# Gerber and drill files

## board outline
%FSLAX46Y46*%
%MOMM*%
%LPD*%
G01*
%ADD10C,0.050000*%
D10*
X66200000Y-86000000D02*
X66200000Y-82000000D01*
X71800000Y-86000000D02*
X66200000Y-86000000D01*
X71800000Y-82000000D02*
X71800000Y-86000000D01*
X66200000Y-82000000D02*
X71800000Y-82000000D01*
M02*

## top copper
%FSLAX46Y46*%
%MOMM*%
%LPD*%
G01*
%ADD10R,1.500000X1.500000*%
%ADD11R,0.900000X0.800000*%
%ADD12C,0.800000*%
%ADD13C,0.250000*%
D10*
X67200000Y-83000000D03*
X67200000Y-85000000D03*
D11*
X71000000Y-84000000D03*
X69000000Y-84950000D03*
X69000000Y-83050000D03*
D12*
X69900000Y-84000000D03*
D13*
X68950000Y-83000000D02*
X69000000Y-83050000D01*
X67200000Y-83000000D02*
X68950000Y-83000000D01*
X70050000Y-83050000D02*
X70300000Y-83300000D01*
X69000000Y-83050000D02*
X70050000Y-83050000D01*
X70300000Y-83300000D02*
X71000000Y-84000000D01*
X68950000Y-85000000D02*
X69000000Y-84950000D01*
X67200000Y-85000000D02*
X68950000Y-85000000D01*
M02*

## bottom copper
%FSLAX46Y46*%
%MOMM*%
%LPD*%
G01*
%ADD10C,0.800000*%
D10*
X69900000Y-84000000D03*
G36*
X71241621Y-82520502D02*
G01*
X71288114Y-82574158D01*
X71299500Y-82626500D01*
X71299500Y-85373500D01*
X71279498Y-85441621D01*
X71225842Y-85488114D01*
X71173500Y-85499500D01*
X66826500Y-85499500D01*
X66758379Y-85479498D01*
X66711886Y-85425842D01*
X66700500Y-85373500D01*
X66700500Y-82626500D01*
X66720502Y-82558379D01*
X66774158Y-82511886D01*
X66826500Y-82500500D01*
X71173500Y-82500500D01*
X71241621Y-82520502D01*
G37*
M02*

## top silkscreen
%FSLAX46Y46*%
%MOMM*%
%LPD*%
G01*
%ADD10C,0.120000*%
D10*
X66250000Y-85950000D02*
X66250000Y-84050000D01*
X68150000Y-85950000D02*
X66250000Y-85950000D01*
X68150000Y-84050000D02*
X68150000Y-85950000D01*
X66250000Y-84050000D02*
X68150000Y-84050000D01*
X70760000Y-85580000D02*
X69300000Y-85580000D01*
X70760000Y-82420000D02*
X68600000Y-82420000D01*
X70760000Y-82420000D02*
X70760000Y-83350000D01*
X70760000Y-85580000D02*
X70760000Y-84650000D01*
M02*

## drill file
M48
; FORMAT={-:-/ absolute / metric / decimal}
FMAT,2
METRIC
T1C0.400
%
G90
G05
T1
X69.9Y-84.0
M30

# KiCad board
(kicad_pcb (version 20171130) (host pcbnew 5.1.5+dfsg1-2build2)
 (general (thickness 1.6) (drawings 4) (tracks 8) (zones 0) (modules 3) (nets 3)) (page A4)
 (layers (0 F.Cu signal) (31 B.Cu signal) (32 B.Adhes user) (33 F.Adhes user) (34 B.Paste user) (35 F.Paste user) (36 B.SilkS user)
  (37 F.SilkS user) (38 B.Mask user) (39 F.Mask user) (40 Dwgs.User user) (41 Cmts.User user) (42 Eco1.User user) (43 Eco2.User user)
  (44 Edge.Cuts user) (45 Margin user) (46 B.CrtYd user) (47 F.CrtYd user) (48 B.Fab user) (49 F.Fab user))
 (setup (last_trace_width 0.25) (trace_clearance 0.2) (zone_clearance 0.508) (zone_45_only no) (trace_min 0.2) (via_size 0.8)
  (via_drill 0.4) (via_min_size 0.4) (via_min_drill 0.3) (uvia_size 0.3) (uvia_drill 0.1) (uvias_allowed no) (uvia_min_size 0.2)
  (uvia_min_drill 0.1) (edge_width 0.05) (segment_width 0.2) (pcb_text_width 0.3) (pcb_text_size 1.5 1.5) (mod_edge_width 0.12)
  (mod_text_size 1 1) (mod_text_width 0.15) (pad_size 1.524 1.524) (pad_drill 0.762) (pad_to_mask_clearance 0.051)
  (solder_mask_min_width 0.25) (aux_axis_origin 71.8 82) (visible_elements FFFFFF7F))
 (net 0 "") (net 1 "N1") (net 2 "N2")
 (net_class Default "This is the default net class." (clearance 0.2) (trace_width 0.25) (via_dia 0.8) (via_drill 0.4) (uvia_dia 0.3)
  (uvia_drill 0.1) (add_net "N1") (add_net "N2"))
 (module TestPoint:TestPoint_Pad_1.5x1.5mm (layer F.Cu) (at 67.2 83)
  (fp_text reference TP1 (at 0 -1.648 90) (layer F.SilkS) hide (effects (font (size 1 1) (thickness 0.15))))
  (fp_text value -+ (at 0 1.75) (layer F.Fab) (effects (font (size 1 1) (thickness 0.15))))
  (pad 1 smd rect (at 0 0) (size 1.5 1.5) (layers F.Cu F.Mask) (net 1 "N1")))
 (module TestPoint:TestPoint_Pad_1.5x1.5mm (layer F.Cu) (at 67.2 85)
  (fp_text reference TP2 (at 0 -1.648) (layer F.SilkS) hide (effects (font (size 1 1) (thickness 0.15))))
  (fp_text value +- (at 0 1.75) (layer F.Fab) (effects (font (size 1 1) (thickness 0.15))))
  (fp_line (start -0.95 0.95) (end -0.95 -0.95) (layer F.SilkS) (width 0.12))
  (fp_line (start 0.95 0.95) (end -0.95 0.95) (layer F.SilkS) (width 0.12))
  (fp_line (start 0.95 -0.95) (end 0.95 0.95) (layer F.SilkS) (width 0.12))
  (fp_line (start -0.95 -0.95) (end 0.95 -0.95) (layer F.SilkS) (width 0.12))
  (pad 1 smd rect (at 0 0) (size 1.5 1.5) (layers F.Cu F.Mask) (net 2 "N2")))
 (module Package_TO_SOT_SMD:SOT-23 (layer F.Cu) (at 70 84)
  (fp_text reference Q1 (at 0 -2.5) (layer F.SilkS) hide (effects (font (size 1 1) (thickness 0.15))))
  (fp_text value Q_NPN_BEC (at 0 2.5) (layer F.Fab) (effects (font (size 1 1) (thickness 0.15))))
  (fp_line (start 0.76 1.58) (end -0.7 1.58) (layer F.SilkS) (width 0.12))
  (fp_line (start 0.76 -1.58) (end -1.4 -1.58) (layer F.SilkS) (width 0.12))
  (fp_line (start 0.76 -1.58) (end 0.76 -0.65) (layer F.SilkS) (width 0.12))
  (fp_line (start 0.76 1.58) (end 0.76 0.65) (layer F.SilkS) (width 0.12))
  (pad 3 smd rect (at 1 0) (size 0.9 0.8) (layers F.Cu F.Paste F.Mask) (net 1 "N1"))
  (pad 2 smd rect (at -1 0.95) (size 0.9 0.8) (layers F.Cu F.Paste F.Mask) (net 2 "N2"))
  (pad 1 smd rect (at -1 -0.95) (size 0.9 0.8) (layers F.Cu F.Paste F.Mask) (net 1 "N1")))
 (gr_line (start 66.2 86) (end 66.2 82) (layer Edge.Cuts) (width 0.05))
 (gr_line (start 71.8 86) (end 66.2 86) (layer Edge.Cuts) (width 0.05))
 (gr_line (start 71.8 82) (end 71.8 86) (layer Edge.Cuts) (width 0.05))
 (gr_line (start 66.2 82) (end 71.8 82) (layer Edge.Cuts) (width 0.05))
 (segment (start 68.95 83) (end 69 83.05) (width 0.25) (layer F.Cu) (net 1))
 (segment (start 67.2 83) (end 68.95 83) (width 0.25) (layer F.Cu) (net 1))
 (segment (start 70.05 83.05) (end 70.3 83.3) (width 0.25) (layer F.Cu) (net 1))
 (segment (start 69 83.05) (end 70.05 83.05) (width 0.25) (layer F.Cu) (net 1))
 (segment (start 70.3 83.3) (end 71 84) (width 0.25) (layer F.Cu) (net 1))
 (via (at 69.9 84) (size 0.8) (drill 0.4) (layers F.Cu B.Cu) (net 1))
 (segment (start 68.95 85) (end 69 84.95) (width 0.25) (layer F.Cu) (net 2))
 (segment (start 67.2 85) (end 68.95 85) (width 0.25) (layer F.Cu) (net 2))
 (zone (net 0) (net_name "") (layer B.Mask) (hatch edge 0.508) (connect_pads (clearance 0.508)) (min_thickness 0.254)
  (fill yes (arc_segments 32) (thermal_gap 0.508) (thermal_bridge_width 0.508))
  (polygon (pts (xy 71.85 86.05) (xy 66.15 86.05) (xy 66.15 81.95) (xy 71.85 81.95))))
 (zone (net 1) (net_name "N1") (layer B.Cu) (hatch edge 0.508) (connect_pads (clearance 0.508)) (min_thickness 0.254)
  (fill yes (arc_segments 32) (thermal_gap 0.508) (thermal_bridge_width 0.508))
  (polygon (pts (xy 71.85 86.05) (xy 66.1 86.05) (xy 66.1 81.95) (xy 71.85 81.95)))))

